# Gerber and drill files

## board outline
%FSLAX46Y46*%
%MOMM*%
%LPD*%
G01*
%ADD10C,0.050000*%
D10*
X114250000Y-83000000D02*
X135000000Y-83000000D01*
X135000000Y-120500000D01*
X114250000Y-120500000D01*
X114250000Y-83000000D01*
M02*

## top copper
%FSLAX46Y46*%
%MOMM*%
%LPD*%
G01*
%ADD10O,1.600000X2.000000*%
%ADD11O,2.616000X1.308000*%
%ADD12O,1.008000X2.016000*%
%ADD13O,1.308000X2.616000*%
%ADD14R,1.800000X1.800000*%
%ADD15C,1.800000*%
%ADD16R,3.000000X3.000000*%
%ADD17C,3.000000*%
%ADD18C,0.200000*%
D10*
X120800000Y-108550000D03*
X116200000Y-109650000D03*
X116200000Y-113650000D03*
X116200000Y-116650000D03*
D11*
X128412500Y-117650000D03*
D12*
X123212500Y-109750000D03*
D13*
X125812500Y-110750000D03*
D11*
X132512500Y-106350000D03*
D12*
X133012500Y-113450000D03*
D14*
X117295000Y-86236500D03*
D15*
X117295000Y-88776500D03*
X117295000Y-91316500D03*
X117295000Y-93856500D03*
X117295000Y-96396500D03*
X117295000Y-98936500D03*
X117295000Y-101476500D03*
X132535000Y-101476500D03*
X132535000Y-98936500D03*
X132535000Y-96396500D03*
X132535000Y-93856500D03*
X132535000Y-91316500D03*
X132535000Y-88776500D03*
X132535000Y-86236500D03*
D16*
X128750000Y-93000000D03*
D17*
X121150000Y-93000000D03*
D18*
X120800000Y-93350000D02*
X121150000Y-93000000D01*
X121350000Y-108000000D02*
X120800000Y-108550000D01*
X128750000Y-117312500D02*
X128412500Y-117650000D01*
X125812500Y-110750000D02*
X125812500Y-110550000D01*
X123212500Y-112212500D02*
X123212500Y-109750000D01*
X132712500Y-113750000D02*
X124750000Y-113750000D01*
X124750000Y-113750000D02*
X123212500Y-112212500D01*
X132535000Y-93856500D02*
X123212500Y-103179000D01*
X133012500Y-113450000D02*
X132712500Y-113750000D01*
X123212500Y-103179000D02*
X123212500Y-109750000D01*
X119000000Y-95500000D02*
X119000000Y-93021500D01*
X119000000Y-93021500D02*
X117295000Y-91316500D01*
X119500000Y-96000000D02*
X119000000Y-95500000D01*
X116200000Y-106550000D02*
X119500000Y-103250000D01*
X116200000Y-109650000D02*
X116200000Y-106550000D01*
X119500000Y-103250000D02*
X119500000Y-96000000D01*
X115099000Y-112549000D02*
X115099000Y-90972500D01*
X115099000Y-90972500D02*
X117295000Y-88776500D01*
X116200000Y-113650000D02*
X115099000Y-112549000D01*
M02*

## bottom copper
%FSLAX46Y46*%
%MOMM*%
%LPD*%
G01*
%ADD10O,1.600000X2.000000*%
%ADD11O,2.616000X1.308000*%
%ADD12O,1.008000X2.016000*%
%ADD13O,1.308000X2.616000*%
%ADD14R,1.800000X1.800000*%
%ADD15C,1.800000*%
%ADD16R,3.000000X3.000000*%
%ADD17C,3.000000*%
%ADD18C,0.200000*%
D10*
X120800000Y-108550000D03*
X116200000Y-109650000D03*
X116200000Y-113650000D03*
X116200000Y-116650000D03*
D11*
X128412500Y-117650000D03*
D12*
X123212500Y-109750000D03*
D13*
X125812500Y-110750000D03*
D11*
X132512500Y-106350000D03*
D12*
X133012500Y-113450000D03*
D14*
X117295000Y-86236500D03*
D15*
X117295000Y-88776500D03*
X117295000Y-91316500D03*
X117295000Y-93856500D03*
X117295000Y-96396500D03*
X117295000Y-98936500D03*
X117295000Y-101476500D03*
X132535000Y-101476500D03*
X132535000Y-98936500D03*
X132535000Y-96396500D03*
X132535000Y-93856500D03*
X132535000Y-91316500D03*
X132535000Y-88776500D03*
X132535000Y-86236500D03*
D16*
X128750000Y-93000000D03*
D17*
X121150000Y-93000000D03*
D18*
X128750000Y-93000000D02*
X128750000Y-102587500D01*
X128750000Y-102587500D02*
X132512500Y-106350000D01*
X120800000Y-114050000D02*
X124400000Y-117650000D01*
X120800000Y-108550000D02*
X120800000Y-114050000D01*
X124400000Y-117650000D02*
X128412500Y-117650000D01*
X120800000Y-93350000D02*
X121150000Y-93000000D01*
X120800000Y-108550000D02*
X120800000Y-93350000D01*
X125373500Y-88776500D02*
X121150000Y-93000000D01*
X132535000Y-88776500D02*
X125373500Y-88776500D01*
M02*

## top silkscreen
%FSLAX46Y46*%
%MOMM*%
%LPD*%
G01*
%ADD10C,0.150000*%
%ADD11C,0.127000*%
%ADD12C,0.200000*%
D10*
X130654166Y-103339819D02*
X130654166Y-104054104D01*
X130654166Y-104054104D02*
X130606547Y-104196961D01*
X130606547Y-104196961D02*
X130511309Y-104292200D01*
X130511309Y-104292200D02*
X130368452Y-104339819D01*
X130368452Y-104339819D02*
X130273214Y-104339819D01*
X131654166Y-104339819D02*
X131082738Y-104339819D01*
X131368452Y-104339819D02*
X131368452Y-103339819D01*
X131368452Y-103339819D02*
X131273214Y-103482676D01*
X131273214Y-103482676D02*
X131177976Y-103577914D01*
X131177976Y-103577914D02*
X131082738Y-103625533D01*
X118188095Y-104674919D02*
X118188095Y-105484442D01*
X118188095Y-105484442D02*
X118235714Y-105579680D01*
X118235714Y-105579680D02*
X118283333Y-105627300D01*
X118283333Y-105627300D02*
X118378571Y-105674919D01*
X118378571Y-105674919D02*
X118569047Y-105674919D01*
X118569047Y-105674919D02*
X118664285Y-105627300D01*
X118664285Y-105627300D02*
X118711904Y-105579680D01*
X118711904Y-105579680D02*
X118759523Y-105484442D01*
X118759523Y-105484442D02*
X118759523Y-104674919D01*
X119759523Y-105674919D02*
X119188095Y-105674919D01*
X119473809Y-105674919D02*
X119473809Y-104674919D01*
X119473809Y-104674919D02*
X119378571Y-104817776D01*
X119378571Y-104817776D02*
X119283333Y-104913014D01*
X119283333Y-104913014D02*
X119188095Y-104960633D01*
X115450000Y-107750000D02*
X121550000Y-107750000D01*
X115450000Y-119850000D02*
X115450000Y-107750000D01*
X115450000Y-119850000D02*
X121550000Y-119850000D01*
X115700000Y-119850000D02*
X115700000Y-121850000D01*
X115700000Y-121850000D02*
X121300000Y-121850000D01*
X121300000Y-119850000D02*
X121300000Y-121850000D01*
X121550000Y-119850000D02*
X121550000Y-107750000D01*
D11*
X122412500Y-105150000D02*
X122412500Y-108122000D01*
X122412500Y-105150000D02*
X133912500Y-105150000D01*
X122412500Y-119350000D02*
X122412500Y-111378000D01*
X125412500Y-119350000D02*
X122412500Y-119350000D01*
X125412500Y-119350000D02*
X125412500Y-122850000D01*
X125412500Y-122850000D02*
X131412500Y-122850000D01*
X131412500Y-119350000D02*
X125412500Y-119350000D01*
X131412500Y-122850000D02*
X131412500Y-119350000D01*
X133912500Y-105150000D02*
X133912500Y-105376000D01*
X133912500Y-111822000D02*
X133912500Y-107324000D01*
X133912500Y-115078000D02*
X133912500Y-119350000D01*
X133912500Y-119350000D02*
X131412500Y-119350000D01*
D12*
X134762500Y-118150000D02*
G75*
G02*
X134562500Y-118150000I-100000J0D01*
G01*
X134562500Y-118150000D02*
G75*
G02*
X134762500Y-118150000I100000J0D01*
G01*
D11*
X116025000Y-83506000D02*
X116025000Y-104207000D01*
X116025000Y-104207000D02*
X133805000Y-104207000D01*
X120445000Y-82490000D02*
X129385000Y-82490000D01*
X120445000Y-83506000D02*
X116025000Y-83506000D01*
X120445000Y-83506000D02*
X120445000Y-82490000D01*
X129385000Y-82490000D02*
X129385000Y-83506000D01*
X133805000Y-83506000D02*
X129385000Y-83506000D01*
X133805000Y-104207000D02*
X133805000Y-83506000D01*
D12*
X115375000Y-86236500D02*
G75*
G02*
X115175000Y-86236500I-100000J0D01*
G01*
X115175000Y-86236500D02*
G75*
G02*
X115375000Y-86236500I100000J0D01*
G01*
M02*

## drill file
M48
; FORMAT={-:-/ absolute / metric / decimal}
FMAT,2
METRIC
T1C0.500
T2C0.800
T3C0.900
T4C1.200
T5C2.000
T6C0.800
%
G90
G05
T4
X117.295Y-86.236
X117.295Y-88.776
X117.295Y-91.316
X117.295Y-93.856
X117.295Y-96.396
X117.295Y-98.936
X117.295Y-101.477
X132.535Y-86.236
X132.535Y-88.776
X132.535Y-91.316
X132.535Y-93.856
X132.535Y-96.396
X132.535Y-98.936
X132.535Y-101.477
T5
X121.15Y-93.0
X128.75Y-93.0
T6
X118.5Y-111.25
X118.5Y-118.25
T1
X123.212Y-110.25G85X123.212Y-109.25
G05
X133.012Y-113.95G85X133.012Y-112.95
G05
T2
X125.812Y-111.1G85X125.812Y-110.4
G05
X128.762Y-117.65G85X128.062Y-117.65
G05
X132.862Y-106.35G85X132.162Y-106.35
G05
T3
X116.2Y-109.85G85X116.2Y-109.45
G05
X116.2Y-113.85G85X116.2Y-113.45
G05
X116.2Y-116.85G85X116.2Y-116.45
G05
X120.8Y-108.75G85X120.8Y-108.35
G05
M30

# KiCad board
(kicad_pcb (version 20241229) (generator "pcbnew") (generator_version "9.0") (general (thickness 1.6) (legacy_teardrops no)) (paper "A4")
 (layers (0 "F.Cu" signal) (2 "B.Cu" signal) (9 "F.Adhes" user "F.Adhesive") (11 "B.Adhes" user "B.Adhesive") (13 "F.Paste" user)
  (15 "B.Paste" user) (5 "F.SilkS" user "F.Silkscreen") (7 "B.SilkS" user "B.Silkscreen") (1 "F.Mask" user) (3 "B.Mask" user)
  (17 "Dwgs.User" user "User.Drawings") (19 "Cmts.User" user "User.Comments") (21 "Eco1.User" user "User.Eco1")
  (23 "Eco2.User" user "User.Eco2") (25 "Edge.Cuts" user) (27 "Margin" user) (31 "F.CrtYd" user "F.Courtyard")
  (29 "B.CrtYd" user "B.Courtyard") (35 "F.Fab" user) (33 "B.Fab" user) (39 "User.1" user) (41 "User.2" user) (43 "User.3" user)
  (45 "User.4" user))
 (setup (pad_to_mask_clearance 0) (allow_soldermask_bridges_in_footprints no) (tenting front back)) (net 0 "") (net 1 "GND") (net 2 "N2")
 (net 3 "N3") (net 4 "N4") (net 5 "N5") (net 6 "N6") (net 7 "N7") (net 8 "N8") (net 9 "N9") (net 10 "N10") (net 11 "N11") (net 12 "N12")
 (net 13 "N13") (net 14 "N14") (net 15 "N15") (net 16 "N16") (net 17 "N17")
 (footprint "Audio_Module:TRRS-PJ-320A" (layer "F.Cu") (at 118.5 119.85 180)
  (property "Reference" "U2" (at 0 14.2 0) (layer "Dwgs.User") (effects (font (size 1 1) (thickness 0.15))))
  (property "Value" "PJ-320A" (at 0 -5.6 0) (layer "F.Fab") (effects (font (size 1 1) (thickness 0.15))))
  (fp_line (start 3.05 12.1) (end -3.05 12.1) (stroke (width 0.15) (type solid)) (layer "F.SilkS"))
  (fp_line (start 3.05 0) (end 3.05 12.1) (stroke (width 0.15) (type solid)) (layer "F.SilkS"))
  (fp_line (start 3.05 0) (end -3.05 0) (stroke (width 0.15) (type solid)) (layer "F.SilkS"))
  (fp_line (start 2.8 0) (end 2.8 -2) (stroke (width 0.15) (type solid)) (layer "F.SilkS"))
  (fp_line (start 2.8 -2) (end -2.8 -2) (stroke (width 0.15) (type solid)) (layer "F.SilkS"))
  (fp_line (start -2.8 0) (end -2.8 -2) (stroke (width 0.15) (type solid)) (layer "F.SilkS"))
  (fp_line (start -3.05 0) (end -3.05 12.1) (stroke (width 0.15) (type solid)) (layer "F.SilkS"))
  (pad "" np_thru_hole circle (at 0 1.6 180) (size 0.8 0.8) (drill 0.8) (layers "*.Cu" "*.Mask"))
  (pad "" np_thru_hole circle (at 0 8.6 180) (size 0.8 0.8) (drill 0.8) (layers "*.Cu" "*.Mask"))
  (pad "1" thru_hole oval (at -2.3 11.3 180) (size 1.6 2) (drill oval 0.9 1.3) (layers "*.Cu" "*.Mask") (remove_unused_layers no)
   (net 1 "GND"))
  (pad "2" thru_hole oval (at 2.3 10.2 180) (size 1.6 2) (drill oval 0.9 1.3) (layers "*.Cu" "*.Mask") (remove_unused_layers no)
   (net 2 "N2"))
  (pad "3" thru_hole oval (at 2.3 6.2 180) (size 1.6 2) (drill oval 0.9 1.3) (layers "*.Cu" "*.Mask") (remove_unused_layers no) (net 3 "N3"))
  (pad "4" thru_hole oval (at 2.3 3.2 180) (size 1.6 2) (drill oval 0.9 1.3) (layers "*.Cu" "*.Mask") (remove_unused_layers no) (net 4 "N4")))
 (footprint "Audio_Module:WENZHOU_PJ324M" (layer "F.Cu") (at 128.4125 112.25 180)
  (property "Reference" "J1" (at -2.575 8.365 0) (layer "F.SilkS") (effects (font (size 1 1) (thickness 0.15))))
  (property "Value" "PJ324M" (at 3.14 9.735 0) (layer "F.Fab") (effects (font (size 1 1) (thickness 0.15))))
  (fp_line (start 6 7.1) (end 6 4.128) (stroke (width 0.127) (type solid)) (layer "F.SilkS"))
  (fp_line (start 6 7.1) (end -5.5 7.1) (stroke (width 0.127) (type solid)) (layer "F.SilkS"))
  (fp_line (start 6 -7.1) (end 6 0.872) (stroke (width 0.127) (type solid)) (layer "F.SilkS"))
  (fp_line (start 3 -7.1) (end 6 -7.1) (stroke (width 0.127) (type solid)) (layer "F.SilkS"))
  (fp_line (start 3 -7.1) (end 3 -10.6) (stroke (width 0.127) (type solid)) (layer "F.SilkS"))
  (fp_line (start 3 -10.6) (end -3 -10.6) (stroke (width 0.127) (type solid)) (layer "F.SilkS"))
  (fp_line (start -3 -7.1) (end 3 -7.1) (stroke (width 0.127) (type solid)) (layer "F.SilkS"))
  (fp_line (start -3 -10.6) (end -3 -7.1) (stroke (width 0.127) (type solid)) (layer "F.SilkS"))
  (fp_line (start -5.5 7.1) (end -5.5 6.874) (stroke (width 0.127) (type solid)) (layer "F.SilkS"))
  (fp_line (start -5.5 0.428) (end -5.5 4.926) (stroke (width 0.127) (type solid)) (layer "F.SilkS"))
  (fp_line (start -5.5 -2.828) (end -5.5 -7.1) (stroke (width 0.127) (type solid)) (layer "F.SilkS"))
  (fp_line (start -5.5 -7.1) (end -3 -7.1) (stroke (width 0.127) (type solid)) (layer "F.SilkS"))
  (fp_circle (center -6.25 -5.9) (end -6.15 -5.9) (stroke (width 0.2) (type solid)) (fill no) (layer "F.SilkS"))
  (pad "1" thru_hole oval (at 0 -5.4 180) (size 2.616 1.308) (drill oval 1.5 0.8) (layers "*.Cu" "*.Mask") (remove_unused_layers no)
   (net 1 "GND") (solder_mask_margin 0.102))
  (pad "2" thru_hole oval (at 5.2 2.5 180) (size 1.008 2.016) (drill oval 0.5 1.5) (layers "*.Cu" "*.Mask") (remove_unused_layers no)
   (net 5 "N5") (solder_mask_margin 0.102))
  (pad "3" thru_hole oval (at 2.6 1.5 180) (size 1.308 2.616) (drill oval 0.8 1.5) (layers "*.Cu" "*.Mask") (remove_unused_layers no)
   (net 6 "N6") (solder_mask_margin 0.102))
  (pad "4" thru_hole oval (at -4.1 5.9 180) (size 2.616 1.308) (drill oval 1.5 0.8) (layers "*.Cu" "*.Mask") (remove_unused_layers no)
   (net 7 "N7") (solder_mask_margin 0.102))
  (pad "5" thru_hole oval (at -4.6 -1.2 180) (size 1.008 2.016) (drill oval 0.5 1.5) (layers "*.Cu" "*.Mask") (remove_unused_layers no)
   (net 5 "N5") (solder_mask_margin 0.102)))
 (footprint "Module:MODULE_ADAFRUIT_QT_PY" (layer "F.Cu") (at 124.915 93.8565)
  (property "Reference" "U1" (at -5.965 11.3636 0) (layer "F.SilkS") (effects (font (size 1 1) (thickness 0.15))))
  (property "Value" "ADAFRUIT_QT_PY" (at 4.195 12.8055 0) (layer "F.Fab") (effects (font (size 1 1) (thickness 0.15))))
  (fp_line (start -8.89 -10.3505) (end -8.89 10.3505) (stroke (width 0.127) (type solid)) (layer "F.SilkS"))
  (fp_line (start -8.89 10.3505) (end 8.89 10.3505) (stroke (width 0.127) (type solid)) (layer "F.SilkS"))
  (fp_line (start -4.47 -11.3665) (end 4.47 -11.3665) (stroke (width 0.127) (type solid)) (layer "F.SilkS"))
  (fp_line (start -4.47 -10.3505) (end -8.89 -10.3505) (stroke (width 0.127) (type solid)) (layer "F.SilkS"))
  (fp_line (start -4.47 -10.3505) (end -4.47 -11.3665) (stroke (width 0.127) (type solid)) (layer "F.SilkS"))
  (fp_line (start 4.47 -11.3665) (end 4.47 -10.3505) (stroke (width 0.127) (type solid)) (layer "F.SilkS"))
  (fp_line (start 8.89 -10.3505) (end 4.47 -10.3505) (stroke (width 0.127) (type solid)) (layer "F.SilkS"))
  (fp_line (start 8.89 10.3505) (end 8.89 -10.3505) (stroke (width 0.127) (type solid)) (layer "F.SilkS"))
  (fp_circle (center -9.64 -7.62) (end -9.54 -7.62) (stroke (width 0.2) (type solid)) (fill no) (layer "F.SilkS"))
  (pad "1" thru_hole rect (at -7.62 -7.62) (size 1.8 1.8) (drill 1.2) (layers "*.Cu" "*.Mask") (remove_unused_layers no) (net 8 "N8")
   (solder_mask_margin 0.102))
  (pad "2" thru_hole circle (at -7.62 -5.08) (size 1.8 1.8) (drill 1.2) (layers "*.Cu" "*.Mask") (remove_unused_layers no) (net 3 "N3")
   (solder_mask_margin 0.102))
  (pad "3" thru_hole circle (at -7.62 -2.54) (size 1.8 1.8) (drill 1.2) (layers "*.Cu" "*.Mask") (remove_unused_layers no) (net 2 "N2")
   (solder_mask_margin 0.102))
  (pad "4" thru_hole circle (at -7.62 0) (size 1.8 1.8) (drill 1.2) (layers "*.Cu" "*.Mask") (remove_unused_layers no) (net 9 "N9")
   (solder_mask_margin 0.102))
  (pad "5" thru_hole circle (at -7.62 2.54) (size 1.8 1.8) (drill 1.2) (layers "*.Cu" "*.Mask") (remove_unused_layers no) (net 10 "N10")
   (solder_mask_margin 0.102))
  (pad "6" thru_hole circle (at -7.62 5.08) (size 1.8 1.8) (drill 1.2) (layers "*.Cu" "*.Mask") (remove_unused_layers no) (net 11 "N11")
   (solder_mask_margin 0.102))
  (pad "7" thru_hole circle (at -7.62 7.62) (size 1.8 1.8) (drill 1.2) (layers "*.Cu" "*.Mask") (remove_unused_layers no) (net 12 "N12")
   (solder_mask_margin 0.102))
  (pad "8" thru_hole circle (at 7.62 7.62) (size 1.8 1.8) (drill 1.2) (layers "*.Cu" "*.Mask") (remove_unused_layers no) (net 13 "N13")
   (solder_mask_margin 0.102))
  (pad "9" thru_hole circle (at 7.62 5.08) (size 1.8 1.8) (drill 1.2) (layers "*.Cu" "*.Mask") (remove_unused_layers no) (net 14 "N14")
   (solder_mask_margin 0.102))
  (pad "10" thru_hole circle (at 7.62 2.54) (size 1.8 1.8) (drill 1.2) (layers "*.Cu" "*.Mask") (remove_unused_layers no) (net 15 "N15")
   (solder_mask_margin 0.102))
  (pad "11" thru_hole circle (at 7.62 0) (size 1.8 1.8) (drill 1.2) (layers "*.Cu" "*.Mask") (remove_unused_layers no) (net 5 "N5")
   (solder_mask_margin 0.102))
  (pad "12" thru_hole circle (at 7.62 -2.54) (size 1.8 1.8) (drill 1.2) (layers "*.Cu" "*.Mask") (remove_unused_layers no) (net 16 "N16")
   (solder_mask_margin 0.102))
  (pad "13" thru_hole circle (at 7.62 -5.08) (size 1.8 1.8) (drill 1.2) (layers "*.Cu" "*.Mask") (remove_unused_layers no) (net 1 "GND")
   (solder_mask_margin 0.102))
  (pad "14" thru_hole circle (at 7.62 -7.62) (size 1.8 1.8) (drill 1.2) (layers "*.Cu" "*.Mask") (remove_unused_layers no) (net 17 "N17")
   (solder_mask_margin 0.102)))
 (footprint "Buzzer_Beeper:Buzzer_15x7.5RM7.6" (layer "B.Cu") (at 128.75 93 180)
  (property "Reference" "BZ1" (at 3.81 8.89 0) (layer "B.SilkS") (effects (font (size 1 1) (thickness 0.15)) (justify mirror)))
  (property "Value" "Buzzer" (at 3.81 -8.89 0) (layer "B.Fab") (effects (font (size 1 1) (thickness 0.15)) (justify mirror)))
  (pad "1" thru_hole rect (at 0 0 180) (size 3 3) (drill 2) (layers "*.Cu" "*.Mask") (remove_unused_layers no) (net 7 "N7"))
  (pad "2" thru_hole circle (at 7.6 0 180) (size 3 3) (drill 2) (layers "*.Cu" "*.Mask") (remove_unused_layers no) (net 1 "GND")))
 (gr_rect (start 114.25 83) (end 135 120.5) (stroke (width 0.05) (type default)) (fill no) (layer "Edge.Cuts"))
 (segment (start 128.75 93) (end 128.75 102.5875) (width 0.2) (layer "B.Cu") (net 7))
 (segment (start 128.75 102.5875) (end 132.5125 106.35) (width 0.2) (layer "B.Cu") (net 7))
 (segment (start 120.8 93.35) (end 121.15 93) (width 0.2) (layer "F.Cu") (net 1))
 (segment (start 121.35 108) (end 120.8 108.55) (width 0.2) (layer "F.Cu") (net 1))
 (segment (start 128.75 117.3125) (end 128.4125 117.65) (width 0.2) (layer "F.Cu") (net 1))
 (segment (start 120.8 114.05) (end 124.4 117.65) (width 0.2) (layer "B.Cu") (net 1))
 (segment (start 120.8 108.55) (end 120.8 114.05) (width 0.2) (layer "B.Cu") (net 1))
 (segment (start 124.4 117.65) (end 128.4125 117.65) (width 0.2) (layer "B.Cu") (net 1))
 (segment (start 120.8 93.35) (end 121.15 93) (width 0.2) (layer "B.Cu") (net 1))
 (segment (start 120.8 108.55) (end 120.8 93.35) (width 0.2) (layer "B.Cu") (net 1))
 (segment (start 125.3735 88.7765) (end 121.15 93) (width 0.2) (layer "B.Cu") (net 1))
 (segment (start 132.535 88.7765) (end 125.3735 88.7765) (width 0.2) (layer "B.Cu") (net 1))
 (segment (start 125.8125 110.75) (end 125.8125 110.55) (width 0.2) (layer "F.Cu") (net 6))
 (segment (start 123.2125 112.2125) (end 123.2125 109.75) (width 0.2) (layer "F.Cu") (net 5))
 (segment (start 132.7125 113.75) (end 124.75 113.75) (width 0.2) (layer "F.Cu") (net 5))
 (segment (start 124.75 113.75) (end 123.2125 112.2125) (width 0.2) (layer "F.Cu") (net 5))
 (segment (start 132.535 93.8565) (end 123.2125 103.179) (width 0.2) (layer "F.Cu") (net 5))
 (segment (start 133.0125 113.45) (end 132.7125 113.75) (width 0.2) (layer "F.Cu") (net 5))
 (segment (start 123.2125 103.179) (end 123.2125 109.75) (width 0.2) (layer "F.Cu") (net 5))
 (segment (start 119 95.5) (end 119 93.0215) (width 0.2) (layer "F.Cu") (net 2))
 (segment (start 119 93.0215) (end 117.295 91.3165) (width 0.2) (layer "F.Cu") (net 2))
 (segment (start 119.5 96) (end 119 95.5) (width 0.2) (layer "F.Cu") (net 2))
 (segment (start 116.2 106.55) (end 119.5 103.25) (width 0.2) (layer "F.Cu") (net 2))
 (segment (start 116.2 109.65) (end 116.2 106.55) (width 0.2) (layer "F.Cu") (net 2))
 (segment (start 119.5 103.25) (end 119.5 96) (width 0.2) (layer "F.Cu") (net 2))
 (segment (start 115.099 112.549) (end 115.099 90.9725) (width 0.2) (layer "F.Cu") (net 3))
 (segment (start 115.099 90.9725) (end 117.295 88.7765) (width 0.2) (layer "F.Cu") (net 3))
 (segment (start 116.2 113.65) (end 115.099 112.549) (width 0.2) (layer "F.Cu") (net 3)))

